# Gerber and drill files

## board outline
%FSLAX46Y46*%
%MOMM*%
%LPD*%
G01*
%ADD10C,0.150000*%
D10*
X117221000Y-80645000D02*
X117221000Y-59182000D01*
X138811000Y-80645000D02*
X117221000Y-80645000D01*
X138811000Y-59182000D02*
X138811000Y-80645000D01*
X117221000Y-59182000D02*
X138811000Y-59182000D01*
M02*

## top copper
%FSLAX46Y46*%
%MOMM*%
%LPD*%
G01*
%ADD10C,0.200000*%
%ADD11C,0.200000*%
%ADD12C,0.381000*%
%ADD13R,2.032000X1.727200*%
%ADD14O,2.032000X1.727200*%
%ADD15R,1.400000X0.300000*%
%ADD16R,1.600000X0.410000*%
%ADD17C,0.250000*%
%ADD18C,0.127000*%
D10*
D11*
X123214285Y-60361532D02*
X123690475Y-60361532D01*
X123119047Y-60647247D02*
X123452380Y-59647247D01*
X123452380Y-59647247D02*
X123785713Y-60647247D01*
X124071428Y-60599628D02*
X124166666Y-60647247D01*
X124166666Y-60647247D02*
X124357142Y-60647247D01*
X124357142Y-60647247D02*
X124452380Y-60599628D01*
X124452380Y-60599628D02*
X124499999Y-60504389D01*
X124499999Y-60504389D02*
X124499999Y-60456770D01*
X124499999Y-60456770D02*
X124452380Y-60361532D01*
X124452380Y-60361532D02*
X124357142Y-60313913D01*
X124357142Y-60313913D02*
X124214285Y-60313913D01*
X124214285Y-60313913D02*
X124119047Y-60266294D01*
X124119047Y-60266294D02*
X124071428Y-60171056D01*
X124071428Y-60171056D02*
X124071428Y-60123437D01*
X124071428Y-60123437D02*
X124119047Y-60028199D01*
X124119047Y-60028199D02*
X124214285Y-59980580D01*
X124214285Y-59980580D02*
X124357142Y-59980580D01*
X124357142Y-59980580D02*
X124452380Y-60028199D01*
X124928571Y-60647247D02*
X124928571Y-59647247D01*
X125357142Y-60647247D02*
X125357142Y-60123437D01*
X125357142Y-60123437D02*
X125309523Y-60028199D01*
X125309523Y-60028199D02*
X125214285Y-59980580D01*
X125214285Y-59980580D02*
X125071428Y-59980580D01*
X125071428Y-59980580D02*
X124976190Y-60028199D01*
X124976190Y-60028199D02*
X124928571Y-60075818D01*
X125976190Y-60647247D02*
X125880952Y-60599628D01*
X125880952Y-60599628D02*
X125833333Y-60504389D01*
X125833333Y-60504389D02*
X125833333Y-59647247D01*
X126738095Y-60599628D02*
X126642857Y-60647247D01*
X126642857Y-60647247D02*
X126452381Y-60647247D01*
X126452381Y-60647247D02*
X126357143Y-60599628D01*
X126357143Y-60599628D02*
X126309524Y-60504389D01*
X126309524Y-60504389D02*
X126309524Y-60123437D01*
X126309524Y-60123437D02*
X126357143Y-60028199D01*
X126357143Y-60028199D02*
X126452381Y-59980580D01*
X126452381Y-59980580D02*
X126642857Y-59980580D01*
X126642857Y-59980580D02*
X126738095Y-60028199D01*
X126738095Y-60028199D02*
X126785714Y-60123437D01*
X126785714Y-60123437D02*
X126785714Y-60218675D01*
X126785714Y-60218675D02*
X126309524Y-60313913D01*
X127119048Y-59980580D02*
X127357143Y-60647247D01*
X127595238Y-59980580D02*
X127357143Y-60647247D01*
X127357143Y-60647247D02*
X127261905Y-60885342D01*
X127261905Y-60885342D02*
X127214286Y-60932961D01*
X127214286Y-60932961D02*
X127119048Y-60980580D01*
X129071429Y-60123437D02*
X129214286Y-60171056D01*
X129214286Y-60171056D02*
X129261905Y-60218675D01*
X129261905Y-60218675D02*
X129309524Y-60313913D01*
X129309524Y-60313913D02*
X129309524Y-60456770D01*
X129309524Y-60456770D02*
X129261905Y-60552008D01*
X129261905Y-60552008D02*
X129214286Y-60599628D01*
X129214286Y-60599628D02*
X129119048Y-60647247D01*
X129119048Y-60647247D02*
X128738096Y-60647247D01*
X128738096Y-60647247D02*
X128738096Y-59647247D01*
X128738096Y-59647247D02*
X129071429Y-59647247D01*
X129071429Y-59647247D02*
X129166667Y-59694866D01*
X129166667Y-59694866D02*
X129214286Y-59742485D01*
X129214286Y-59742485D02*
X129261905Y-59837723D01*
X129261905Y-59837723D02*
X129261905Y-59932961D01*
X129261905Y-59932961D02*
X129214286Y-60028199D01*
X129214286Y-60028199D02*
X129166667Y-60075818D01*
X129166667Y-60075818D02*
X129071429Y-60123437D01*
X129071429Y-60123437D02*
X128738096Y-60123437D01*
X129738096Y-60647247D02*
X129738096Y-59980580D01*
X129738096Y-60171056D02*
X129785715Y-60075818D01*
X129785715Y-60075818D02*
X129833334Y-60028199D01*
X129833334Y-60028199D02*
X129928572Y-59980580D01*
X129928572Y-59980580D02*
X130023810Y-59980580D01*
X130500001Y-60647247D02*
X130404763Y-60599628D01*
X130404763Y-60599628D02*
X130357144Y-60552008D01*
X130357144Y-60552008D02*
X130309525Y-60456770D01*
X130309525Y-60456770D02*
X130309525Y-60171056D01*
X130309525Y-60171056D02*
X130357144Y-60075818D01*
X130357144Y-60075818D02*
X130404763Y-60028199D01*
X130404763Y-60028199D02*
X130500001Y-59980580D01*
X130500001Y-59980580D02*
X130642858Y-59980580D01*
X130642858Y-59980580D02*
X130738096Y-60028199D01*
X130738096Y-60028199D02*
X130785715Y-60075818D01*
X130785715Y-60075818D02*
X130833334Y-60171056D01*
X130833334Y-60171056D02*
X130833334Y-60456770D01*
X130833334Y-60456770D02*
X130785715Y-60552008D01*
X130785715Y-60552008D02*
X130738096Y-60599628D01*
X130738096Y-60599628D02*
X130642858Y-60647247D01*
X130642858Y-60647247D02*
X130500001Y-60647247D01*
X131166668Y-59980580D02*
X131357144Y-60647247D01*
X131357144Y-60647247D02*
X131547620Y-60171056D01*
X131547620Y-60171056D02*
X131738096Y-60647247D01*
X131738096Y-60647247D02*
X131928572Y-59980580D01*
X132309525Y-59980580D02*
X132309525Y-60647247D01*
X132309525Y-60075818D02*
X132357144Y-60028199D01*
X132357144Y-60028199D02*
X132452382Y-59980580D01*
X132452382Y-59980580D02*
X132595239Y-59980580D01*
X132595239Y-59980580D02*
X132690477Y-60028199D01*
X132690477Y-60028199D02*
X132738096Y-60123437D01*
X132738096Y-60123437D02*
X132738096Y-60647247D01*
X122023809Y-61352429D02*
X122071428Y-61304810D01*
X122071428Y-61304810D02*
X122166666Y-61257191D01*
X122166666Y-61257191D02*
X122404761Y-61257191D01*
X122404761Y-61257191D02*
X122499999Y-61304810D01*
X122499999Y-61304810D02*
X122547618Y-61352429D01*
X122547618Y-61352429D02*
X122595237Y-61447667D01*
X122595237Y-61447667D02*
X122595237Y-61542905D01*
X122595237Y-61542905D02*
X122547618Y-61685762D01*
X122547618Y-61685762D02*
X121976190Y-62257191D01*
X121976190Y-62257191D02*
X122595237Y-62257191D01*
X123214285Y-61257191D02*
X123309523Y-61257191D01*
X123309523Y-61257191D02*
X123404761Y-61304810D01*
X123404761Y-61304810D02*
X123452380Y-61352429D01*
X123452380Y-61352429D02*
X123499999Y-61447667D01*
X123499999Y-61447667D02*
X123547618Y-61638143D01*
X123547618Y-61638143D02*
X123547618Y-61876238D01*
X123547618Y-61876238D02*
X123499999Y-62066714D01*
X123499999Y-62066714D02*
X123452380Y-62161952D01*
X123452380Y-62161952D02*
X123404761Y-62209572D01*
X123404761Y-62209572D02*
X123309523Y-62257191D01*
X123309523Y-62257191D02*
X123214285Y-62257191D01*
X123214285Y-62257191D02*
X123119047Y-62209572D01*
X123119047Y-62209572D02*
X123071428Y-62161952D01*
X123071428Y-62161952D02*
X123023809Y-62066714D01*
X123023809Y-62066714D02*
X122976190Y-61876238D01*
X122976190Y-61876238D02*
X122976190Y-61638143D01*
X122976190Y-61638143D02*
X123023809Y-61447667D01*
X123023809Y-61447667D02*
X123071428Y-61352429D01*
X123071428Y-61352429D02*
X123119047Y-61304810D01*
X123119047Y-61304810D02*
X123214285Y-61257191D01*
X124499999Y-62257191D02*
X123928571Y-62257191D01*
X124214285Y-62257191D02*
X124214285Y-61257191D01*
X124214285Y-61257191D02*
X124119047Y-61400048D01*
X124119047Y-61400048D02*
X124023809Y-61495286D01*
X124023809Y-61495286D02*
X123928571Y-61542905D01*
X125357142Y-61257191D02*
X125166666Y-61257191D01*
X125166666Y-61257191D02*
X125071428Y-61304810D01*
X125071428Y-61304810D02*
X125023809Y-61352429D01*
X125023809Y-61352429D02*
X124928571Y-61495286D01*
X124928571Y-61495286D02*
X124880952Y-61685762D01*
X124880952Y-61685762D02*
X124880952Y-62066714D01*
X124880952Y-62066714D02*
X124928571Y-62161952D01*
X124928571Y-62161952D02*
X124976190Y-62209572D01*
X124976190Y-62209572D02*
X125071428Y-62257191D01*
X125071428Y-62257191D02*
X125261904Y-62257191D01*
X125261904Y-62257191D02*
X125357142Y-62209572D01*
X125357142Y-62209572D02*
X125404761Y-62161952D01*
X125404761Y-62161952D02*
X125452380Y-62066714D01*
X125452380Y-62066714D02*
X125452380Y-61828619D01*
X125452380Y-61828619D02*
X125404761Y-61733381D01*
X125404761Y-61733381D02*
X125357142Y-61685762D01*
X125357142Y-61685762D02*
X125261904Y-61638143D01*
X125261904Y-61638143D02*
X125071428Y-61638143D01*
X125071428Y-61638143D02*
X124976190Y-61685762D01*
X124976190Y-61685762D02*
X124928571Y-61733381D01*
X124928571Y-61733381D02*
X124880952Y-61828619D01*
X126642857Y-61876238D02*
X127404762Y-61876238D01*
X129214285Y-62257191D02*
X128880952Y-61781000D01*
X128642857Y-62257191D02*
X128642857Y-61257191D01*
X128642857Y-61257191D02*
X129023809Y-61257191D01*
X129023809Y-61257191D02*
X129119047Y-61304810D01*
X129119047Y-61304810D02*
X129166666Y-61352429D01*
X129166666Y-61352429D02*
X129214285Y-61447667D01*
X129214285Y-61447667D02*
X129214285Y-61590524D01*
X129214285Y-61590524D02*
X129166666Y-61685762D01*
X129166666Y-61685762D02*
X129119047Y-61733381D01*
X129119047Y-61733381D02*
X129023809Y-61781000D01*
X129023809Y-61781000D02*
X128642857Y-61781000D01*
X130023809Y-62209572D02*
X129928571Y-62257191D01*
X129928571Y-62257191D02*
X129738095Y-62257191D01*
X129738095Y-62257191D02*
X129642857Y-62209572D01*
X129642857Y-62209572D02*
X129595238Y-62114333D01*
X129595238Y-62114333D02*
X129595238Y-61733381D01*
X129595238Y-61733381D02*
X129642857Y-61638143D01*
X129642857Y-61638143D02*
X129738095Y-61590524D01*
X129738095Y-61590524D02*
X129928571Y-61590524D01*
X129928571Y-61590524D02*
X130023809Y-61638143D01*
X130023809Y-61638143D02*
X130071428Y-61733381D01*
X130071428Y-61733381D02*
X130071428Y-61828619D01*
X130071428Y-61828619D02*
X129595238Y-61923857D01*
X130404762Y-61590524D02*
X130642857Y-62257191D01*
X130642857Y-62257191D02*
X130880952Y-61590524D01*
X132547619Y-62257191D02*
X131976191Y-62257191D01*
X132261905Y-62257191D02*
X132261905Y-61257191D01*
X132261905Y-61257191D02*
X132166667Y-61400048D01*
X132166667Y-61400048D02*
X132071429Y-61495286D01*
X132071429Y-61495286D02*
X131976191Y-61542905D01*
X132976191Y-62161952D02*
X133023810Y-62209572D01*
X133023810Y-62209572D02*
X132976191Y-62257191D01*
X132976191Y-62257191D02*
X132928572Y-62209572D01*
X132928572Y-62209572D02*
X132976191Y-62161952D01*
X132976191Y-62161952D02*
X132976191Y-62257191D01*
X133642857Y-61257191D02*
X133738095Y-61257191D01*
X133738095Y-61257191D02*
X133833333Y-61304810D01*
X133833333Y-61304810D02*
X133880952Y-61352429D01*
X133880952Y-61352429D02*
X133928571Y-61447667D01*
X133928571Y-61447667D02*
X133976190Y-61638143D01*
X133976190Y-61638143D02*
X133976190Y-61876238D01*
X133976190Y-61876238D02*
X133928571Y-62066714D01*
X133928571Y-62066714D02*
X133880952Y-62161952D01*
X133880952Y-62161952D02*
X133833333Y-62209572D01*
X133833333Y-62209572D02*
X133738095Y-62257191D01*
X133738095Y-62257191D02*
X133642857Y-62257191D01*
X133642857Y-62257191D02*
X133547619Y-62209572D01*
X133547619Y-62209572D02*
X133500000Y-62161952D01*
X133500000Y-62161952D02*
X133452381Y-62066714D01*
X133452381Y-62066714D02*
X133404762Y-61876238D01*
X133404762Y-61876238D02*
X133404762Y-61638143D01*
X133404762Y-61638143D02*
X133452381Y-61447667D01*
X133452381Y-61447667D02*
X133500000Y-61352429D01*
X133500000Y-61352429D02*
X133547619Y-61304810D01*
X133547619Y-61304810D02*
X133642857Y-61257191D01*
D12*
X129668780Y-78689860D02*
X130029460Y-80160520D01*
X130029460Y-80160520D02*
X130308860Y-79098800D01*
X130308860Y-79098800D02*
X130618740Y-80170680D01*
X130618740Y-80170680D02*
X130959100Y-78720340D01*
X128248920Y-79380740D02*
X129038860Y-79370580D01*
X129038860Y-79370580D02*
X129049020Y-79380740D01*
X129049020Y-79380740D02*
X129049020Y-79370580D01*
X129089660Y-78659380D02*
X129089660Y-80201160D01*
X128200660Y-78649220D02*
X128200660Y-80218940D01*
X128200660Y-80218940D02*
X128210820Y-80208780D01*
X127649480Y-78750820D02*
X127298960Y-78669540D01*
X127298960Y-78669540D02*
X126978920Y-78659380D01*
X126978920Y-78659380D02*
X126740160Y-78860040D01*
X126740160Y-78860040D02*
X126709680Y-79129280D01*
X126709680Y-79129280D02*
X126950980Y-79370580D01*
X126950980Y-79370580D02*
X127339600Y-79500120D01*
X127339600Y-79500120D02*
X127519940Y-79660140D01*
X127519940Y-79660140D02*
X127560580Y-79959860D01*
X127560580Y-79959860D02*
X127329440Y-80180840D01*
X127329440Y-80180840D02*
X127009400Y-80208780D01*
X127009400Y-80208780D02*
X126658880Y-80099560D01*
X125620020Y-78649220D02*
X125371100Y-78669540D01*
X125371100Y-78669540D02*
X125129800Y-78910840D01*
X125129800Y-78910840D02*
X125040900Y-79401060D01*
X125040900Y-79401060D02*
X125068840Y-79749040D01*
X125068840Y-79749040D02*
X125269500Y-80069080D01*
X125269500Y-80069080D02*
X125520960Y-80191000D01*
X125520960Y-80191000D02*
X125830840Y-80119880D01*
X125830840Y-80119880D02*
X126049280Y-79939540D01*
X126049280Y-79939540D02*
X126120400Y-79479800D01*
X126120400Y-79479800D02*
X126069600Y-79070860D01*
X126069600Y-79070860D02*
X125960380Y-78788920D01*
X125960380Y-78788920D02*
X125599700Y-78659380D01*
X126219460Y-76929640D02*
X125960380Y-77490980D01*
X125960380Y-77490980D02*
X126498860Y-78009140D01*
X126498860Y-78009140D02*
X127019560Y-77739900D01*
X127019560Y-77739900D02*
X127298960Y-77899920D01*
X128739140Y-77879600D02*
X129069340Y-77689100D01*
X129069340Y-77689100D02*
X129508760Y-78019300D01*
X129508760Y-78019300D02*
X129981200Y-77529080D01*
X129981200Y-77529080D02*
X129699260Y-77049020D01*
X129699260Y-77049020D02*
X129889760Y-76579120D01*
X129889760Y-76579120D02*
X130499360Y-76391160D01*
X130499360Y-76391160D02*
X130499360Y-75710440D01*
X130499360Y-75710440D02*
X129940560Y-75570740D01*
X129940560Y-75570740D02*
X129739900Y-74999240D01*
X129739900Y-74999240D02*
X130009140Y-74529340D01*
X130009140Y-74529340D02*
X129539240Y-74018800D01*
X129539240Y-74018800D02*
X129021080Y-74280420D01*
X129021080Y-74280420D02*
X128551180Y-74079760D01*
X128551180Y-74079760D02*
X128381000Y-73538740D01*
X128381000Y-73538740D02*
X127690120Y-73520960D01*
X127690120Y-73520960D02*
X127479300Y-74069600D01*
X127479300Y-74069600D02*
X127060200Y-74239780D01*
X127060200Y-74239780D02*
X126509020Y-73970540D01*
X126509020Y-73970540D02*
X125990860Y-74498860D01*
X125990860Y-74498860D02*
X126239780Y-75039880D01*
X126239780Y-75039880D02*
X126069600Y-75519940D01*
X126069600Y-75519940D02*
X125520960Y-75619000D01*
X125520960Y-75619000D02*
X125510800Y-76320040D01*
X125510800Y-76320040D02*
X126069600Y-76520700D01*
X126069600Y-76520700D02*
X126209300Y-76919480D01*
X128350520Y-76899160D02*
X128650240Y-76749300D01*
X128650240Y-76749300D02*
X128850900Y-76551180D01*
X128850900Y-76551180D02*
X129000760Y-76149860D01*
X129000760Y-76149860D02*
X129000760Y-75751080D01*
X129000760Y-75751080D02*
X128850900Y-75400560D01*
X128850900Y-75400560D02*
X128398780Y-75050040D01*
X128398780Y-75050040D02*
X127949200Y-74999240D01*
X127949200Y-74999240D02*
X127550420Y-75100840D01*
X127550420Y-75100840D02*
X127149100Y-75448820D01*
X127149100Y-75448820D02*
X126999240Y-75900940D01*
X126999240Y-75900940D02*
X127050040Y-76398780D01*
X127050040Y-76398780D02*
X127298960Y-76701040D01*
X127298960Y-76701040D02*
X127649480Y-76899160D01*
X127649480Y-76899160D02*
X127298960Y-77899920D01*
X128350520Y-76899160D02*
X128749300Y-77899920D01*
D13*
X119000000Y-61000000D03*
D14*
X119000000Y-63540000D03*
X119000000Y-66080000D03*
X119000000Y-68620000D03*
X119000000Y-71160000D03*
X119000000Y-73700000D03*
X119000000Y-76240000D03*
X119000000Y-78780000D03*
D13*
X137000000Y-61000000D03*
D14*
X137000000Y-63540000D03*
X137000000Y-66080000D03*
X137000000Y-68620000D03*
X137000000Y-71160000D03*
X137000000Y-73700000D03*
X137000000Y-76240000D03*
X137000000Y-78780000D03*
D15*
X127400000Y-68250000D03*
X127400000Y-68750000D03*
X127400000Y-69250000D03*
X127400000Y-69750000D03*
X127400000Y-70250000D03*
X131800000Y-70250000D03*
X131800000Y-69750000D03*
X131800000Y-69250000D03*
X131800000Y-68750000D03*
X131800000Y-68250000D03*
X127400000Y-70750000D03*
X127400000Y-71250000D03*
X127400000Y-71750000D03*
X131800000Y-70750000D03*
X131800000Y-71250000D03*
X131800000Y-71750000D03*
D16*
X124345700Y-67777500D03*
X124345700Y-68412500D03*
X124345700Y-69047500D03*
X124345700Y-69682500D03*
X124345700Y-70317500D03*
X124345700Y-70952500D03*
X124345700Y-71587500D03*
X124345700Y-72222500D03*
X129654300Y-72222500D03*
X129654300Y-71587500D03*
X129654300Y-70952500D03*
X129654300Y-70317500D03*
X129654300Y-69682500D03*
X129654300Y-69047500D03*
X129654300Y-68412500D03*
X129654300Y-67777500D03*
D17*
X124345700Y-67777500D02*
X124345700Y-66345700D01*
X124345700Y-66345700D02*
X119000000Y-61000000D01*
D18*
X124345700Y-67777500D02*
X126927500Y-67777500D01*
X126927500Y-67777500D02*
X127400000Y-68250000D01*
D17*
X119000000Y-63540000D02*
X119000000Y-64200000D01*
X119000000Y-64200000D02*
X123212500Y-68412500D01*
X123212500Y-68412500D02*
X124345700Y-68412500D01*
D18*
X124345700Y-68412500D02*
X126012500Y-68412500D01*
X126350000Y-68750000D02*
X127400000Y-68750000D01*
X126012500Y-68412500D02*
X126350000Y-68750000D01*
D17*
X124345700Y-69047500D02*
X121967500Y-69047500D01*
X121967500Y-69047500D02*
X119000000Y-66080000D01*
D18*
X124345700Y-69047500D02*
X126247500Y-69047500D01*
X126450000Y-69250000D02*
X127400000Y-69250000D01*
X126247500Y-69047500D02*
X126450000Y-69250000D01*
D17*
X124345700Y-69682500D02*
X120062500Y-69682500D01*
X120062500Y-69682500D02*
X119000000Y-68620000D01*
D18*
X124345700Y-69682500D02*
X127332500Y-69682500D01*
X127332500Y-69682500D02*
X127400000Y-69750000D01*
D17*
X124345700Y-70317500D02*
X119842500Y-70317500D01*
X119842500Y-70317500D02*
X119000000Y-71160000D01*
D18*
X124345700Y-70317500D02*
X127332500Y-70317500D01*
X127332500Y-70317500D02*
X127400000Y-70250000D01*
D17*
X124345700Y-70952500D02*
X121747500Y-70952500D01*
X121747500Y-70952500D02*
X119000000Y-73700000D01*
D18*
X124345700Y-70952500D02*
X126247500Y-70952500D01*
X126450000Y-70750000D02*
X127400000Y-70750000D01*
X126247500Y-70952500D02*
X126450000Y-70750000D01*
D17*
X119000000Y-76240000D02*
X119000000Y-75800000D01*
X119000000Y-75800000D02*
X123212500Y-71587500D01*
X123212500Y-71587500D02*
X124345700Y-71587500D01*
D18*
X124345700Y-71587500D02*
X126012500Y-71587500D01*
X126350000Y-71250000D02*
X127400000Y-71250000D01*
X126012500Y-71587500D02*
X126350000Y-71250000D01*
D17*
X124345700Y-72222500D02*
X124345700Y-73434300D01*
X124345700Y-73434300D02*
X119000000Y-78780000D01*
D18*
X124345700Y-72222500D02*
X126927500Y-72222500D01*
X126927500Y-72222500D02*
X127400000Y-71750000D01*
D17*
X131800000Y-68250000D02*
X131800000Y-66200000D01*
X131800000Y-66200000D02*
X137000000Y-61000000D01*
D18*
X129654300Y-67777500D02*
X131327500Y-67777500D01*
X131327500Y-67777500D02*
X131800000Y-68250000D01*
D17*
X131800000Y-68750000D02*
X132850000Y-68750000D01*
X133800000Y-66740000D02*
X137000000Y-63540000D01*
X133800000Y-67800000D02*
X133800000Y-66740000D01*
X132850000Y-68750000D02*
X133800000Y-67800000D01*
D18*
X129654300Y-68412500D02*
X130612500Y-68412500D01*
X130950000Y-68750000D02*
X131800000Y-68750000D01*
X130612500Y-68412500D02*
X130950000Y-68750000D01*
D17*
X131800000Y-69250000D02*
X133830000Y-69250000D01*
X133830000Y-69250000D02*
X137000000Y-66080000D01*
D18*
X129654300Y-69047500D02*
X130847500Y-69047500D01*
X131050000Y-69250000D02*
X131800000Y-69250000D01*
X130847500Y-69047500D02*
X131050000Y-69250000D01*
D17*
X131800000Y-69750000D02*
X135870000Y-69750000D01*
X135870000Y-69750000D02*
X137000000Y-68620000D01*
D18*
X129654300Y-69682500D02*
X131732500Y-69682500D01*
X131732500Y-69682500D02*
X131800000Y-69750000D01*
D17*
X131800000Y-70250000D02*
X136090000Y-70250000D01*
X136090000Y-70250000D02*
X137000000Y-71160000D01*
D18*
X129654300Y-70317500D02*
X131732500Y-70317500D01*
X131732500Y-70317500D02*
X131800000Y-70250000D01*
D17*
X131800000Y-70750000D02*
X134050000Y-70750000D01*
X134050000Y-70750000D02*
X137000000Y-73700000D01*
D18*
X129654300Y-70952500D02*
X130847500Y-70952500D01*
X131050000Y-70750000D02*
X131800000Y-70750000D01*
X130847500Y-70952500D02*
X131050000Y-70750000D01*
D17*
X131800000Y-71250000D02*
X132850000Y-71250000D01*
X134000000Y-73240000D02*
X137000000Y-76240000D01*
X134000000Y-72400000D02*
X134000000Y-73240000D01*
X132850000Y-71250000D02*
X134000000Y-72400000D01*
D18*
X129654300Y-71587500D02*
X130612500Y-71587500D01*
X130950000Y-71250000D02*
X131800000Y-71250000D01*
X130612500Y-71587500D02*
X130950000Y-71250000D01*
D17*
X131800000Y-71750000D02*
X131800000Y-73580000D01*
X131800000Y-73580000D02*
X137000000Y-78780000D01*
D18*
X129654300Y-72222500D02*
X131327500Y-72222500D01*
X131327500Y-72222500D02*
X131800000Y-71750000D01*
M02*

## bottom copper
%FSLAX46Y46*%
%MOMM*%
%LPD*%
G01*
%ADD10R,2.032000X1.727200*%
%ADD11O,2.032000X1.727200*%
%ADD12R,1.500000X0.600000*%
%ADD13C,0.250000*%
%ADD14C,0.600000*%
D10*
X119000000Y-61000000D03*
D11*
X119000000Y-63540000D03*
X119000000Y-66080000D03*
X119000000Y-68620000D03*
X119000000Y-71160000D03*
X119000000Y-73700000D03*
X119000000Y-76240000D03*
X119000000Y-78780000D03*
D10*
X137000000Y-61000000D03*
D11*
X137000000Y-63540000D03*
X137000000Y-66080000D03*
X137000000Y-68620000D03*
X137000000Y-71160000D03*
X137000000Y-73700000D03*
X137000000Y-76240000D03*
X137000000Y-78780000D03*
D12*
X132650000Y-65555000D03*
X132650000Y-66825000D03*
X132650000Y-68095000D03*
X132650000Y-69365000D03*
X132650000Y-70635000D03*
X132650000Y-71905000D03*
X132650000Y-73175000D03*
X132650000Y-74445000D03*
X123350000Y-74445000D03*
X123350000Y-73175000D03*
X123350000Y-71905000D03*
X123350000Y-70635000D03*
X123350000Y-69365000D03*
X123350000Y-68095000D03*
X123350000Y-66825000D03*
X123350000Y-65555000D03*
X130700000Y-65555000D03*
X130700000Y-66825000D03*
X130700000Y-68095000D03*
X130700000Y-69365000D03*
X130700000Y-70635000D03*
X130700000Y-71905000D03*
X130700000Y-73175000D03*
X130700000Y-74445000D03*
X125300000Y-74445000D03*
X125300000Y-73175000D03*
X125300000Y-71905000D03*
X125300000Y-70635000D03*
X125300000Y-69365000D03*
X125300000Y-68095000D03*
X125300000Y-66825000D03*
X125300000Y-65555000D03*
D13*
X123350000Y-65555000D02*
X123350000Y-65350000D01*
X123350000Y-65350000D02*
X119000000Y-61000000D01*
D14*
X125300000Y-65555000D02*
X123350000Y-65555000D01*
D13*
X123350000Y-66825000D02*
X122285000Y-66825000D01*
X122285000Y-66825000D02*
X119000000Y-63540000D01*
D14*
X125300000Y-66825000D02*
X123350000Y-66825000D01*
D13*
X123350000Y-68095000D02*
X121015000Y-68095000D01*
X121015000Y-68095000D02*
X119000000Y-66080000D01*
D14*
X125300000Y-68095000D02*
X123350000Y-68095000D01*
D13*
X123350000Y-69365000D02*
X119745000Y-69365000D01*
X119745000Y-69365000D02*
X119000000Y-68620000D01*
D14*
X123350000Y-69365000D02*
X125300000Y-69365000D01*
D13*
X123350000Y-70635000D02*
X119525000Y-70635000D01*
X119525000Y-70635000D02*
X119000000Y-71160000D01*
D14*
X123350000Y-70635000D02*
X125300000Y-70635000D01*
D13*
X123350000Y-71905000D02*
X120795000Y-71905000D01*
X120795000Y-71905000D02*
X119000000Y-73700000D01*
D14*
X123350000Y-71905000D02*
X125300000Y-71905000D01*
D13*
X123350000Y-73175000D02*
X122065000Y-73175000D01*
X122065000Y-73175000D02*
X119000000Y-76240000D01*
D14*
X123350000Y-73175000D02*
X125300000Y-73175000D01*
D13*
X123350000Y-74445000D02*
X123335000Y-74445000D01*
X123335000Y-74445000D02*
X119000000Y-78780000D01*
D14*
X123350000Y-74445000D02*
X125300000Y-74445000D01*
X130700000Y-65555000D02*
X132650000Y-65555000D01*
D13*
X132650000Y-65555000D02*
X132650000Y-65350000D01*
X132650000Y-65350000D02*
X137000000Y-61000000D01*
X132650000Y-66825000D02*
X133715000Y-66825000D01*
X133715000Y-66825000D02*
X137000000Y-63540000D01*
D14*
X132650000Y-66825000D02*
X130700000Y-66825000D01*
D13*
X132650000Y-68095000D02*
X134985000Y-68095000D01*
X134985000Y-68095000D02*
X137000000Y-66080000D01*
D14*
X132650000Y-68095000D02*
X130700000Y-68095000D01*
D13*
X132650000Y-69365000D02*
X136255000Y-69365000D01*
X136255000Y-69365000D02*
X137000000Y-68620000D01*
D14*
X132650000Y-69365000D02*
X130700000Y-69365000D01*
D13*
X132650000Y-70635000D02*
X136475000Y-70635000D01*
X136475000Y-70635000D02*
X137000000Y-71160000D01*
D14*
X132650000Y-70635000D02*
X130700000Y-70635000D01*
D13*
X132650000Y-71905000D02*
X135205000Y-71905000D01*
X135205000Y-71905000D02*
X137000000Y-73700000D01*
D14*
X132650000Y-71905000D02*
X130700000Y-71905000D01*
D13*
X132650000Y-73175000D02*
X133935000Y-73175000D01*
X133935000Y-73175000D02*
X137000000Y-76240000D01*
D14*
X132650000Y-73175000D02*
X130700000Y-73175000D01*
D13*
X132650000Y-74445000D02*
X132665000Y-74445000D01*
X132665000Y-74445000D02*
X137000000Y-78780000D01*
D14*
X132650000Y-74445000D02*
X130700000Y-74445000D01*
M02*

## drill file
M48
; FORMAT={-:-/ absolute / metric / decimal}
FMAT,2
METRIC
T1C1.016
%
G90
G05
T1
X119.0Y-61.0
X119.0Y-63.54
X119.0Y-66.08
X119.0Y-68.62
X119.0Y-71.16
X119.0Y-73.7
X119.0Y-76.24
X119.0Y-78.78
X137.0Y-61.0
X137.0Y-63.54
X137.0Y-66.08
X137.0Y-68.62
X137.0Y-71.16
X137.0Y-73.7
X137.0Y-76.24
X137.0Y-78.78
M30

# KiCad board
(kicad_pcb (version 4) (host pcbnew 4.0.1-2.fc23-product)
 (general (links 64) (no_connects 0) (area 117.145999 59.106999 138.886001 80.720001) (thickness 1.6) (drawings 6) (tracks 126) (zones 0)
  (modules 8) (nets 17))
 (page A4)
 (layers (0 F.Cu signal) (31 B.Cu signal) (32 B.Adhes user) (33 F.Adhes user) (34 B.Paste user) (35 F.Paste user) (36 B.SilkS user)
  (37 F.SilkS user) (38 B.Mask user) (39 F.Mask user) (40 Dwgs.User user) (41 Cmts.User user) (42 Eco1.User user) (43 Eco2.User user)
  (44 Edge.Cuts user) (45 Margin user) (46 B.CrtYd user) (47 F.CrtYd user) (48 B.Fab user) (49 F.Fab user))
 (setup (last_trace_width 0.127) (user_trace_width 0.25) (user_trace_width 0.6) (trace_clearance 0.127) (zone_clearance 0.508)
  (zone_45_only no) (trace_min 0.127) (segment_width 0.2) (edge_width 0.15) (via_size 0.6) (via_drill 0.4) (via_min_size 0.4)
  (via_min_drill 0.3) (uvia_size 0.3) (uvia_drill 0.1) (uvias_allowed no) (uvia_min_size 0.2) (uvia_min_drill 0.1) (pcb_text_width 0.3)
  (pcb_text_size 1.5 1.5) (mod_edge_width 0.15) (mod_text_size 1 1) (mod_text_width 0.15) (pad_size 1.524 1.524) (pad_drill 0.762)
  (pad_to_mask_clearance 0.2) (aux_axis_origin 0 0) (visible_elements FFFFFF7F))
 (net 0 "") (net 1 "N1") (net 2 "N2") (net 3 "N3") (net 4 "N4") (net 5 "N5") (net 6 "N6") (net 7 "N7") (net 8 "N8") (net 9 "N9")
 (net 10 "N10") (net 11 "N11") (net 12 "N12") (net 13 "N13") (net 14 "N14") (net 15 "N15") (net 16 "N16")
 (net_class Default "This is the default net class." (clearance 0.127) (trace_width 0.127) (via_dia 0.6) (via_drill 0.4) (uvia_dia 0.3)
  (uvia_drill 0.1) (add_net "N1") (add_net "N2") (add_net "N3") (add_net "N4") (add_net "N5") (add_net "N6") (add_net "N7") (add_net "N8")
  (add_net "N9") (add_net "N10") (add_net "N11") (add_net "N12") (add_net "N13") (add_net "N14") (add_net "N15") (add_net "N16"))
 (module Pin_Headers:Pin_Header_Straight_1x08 (layer F.Cu) (at 119 61)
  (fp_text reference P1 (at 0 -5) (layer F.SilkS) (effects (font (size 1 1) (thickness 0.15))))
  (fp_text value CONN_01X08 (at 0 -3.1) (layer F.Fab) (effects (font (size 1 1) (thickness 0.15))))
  (pad 1 thru_hole rect (at 0 0) (size 2.032 1.7272) (drill 1.016) (layers *.Cu *.Mask F.SilkS) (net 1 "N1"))
  (pad 2 thru_hole oval (at 0 2.54) (size 2.032 1.7272) (drill 1.016) (layers *.Cu *.Mask F.SilkS) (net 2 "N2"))
  (pad 3 thru_hole oval (at 0 5.08) (size 2.032 1.7272) (drill 1.016) (layers *.Cu *.Mask F.SilkS) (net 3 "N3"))
  (pad 4 thru_hole oval (at 0 7.62) (size 2.032 1.7272) (drill 1.016) (layers *.Cu *.Mask F.SilkS) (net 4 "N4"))
  (pad 5 thru_hole oval (at 0 10.16) (size 2.032 1.7272) (drill 1.016) (layers *.Cu *.Mask F.SilkS) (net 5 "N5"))
  (pad 6 thru_hole oval (at 0 12.7) (size 2.032 1.7272) (drill 1.016) (layers *.Cu *.Mask F.SilkS) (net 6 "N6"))
  (pad 7 thru_hole oval (at 0 15.24) (size 2.032 1.7272) (drill 1.016) (layers *.Cu *.Mask F.SilkS) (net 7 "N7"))
  (pad 8 thru_hole oval (at 0 17.78) (size 2.032 1.7272) (drill 1.016) (layers *.Cu *.Mask F.SilkS) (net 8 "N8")))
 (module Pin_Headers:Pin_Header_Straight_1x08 (layer F.Cu) (at 137 61)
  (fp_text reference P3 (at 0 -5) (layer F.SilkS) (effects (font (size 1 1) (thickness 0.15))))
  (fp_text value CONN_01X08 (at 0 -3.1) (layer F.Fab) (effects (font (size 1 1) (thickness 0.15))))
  (pad 1 thru_hole rect (at 0 0) (size 2.032 1.7272) (drill 1.016) (layers *.Cu *.Mask F.SilkS) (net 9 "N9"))
  (pad 2 thru_hole oval (at 0 2.54) (size 2.032 1.7272) (drill 1.016) (layers *.Cu *.Mask F.SilkS) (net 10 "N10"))
  (pad 3 thru_hole oval (at 0 5.08) (size 2.032 1.7272) (drill 1.016) (layers *.Cu *.Mask F.SilkS) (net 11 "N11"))
  (pad 4 thru_hole oval (at 0 7.62) (size 2.032 1.7272) (drill 1.016) (layers *.Cu *.Mask F.SilkS) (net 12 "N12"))
  (pad 5 thru_hole oval (at 0 10.16) (size 2.032 1.7272) (drill 1.016) (layers *.Cu *.Mask F.SilkS) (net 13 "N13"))
  (pad 6 thru_hole oval (at 0 12.7) (size 2.032 1.7272) (drill 1.016) (layers *.Cu *.Mask F.SilkS) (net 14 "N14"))
  (pad 7 thru_hole oval (at 0 15.24) (size 2.032 1.7272) (drill 1.016) (layers *.Cu *.Mask F.SilkS) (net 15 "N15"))
  (pad 8 thru_hole oval (at 0 17.78) (size 2.032 1.7272) (drill 1.016) (layers *.Cu *.Mask F.SilkS) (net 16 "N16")))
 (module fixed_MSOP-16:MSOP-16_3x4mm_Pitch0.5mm (layer F.Cu) (at 129.6 70)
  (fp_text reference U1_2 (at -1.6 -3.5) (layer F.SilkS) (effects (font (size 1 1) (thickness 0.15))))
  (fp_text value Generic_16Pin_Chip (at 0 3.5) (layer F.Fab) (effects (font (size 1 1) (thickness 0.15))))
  (pad 1 smd rect (at -2.2 -1.75) (size 1.4 0.3) (layers F.Cu F.Paste F.Mask) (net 1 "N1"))
  (pad 2 smd rect (at -2.2 -1.25) (size 1.4 0.3) (layers F.Cu F.Paste F.Mask) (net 2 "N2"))
  (pad 3 smd rect (at -2.2 -0.75) (size 1.4 0.3) (layers F.Cu F.Paste F.Mask) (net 3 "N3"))
  (pad 4 smd rect (at -2.2 -0.25) (size 1.4 0.3) (layers F.Cu F.Paste F.Mask) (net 4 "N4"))
  (pad 5 smd rect (at -2.2 0.25) (size 1.4 0.3) (layers F.Cu F.Paste F.Mask) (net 5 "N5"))
  (pad 12 smd rect (at 2.2 0.25) (size 1.4 0.3) (layers F.Cu F.Paste F.Mask) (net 13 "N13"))
  (pad 13 smd rect (at 2.2 -0.25) (size 1.4 0.3) (layers F.Cu F.Paste F.Mask) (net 12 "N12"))
  (pad 14 smd rect (at 2.2 -0.75) (size 1.4 0.3) (layers F.Cu F.Paste F.Mask) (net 11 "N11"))
  (pad 15 smd rect (at 2.2 -1.25) (size 1.4 0.3) (layers F.Cu F.Paste F.Mask) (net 10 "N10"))
  (pad 16 smd rect (at 2.2 -1.75) (size 1.4 0.3) (layers F.Cu F.Paste F.Mask) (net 9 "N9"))
  (pad 6 smd rect (at -2.2 0.75) (size 1.4 0.3) (layers F.Cu F.Paste F.Mask) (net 6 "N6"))
  (pad 7 smd rect (at -2.2 1.25) (size 1.4 0.3) (layers F.Cu F.Paste F.Mask) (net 7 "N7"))
  (pad 8 smd rect (at -2.2 1.75) (size 1.4 0.3) (layers F.Cu F.Paste F.Mask) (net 8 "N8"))
  (pad 11 smd rect (at 2.2 0.75) (size 1.4 0.3) (layers F.Cu F.Paste F.Mask) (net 14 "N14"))
  (pad 10 smd rect (at 2.2 1.25) (size 1.4 0.3) (layers F.Cu F.Paste F.Mask) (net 15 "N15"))
  (pad 9 smd rect (at 2.2 1.75) (size 1.4 0.3) (layers F.Cu F.Paste F.Mask) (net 16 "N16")))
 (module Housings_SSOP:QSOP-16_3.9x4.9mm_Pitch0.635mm (layer F.Cu) (at 127 70)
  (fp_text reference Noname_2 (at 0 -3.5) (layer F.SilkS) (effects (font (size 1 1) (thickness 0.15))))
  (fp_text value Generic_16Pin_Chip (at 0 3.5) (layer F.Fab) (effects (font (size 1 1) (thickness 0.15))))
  (pad 1 smd rect (at -2.6543 -2.2225) (size 1.6 0.41) (layers F.Cu F.Paste F.Mask) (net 1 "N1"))
  (pad 2 smd rect (at -2.6543 -1.5875) (size 1.6 0.41) (layers F.Cu F.Paste F.Mask) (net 2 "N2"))
  (pad 3 smd rect (at -2.6543 -0.9525) (size 1.6 0.41) (layers F.Cu F.Paste F.Mask) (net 3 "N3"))
  (pad 4 smd rect (at -2.6543 -0.3175) (size 1.6 0.41) (layers F.Cu F.Paste F.Mask) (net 4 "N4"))
  (pad 5 smd rect (at -2.6543 0.3175) (size 1.6 0.41) (layers F.Cu F.Paste F.Mask) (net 5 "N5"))
  (pad 6 smd rect (at -2.6543 0.9525) (size 1.6 0.41) (layers F.Cu F.Paste F.Mask) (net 6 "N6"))
  (pad 7 smd rect (at -2.6543 1.5875) (size 1.6 0.41) (layers F.Cu F.Paste F.Mask) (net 7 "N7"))
  (pad 8 smd rect (at -2.6543 2.2225) (size 1.6 0.41) (layers F.Cu F.Paste F.Mask) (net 8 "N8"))
  (pad 9 smd rect (at 2.6543 2.2225) (size 1.6 0.41) (layers F.Cu F.Paste F.Mask) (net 16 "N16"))
  (pad 10 smd rect (at 2.6543 1.5875) (size 1.6 0.41) (layers F.Cu F.Paste F.Mask) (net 15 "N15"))
  (pad 11 smd rect (at 2.6543 0.9525) (size 1.6 0.41) (layers F.Cu F.Paste F.Mask) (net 14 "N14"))
  (pad 12 smd rect (at 2.6543 0.3175) (size 1.6 0.41) (layers F.Cu F.Paste F.Mask) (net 13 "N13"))
  (pad 13 smd rect (at 2.6543 -0.3175) (size 1.6 0.41) (layers F.Cu F.Paste F.Mask) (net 12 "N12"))
  (pad 14 smd rect (at 2.6543 -0.9525) (size 1.6 0.41) (layers F.Cu F.Paste F.Mask) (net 11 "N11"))
  (pad 15 smd rect (at 2.6543 -1.5875) (size 1.6 0.41) (layers F.Cu F.Paste F.Mask) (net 10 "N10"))
  (pad 16 smd rect (at 2.6543 -2.2225) (size 1.6 0.41) (layers F.Cu F.Paste F.Mask) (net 9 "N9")))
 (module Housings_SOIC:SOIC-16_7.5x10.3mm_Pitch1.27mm (layer B.Cu) (at 128 70 180)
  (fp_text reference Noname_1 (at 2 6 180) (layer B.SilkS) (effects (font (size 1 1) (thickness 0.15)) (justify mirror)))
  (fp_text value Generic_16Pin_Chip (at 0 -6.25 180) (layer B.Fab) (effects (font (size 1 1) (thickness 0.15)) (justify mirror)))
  (pad 1 smd rect (at -4.65 4.445 180) (size 1.5 0.6) (layers B.Cu B.Paste B.Mask) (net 9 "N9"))
  (pad 2 smd rect (at -4.65 3.175 180) (size 1.5 0.6) (layers B.Cu B.Paste B.Mask) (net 10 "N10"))
  (pad 3 smd rect (at -4.65 1.905 180) (size 1.5 0.6) (layers B.Cu B.Paste B.Mask) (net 11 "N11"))
  (pad 4 smd rect (at -4.65 0.635 180) (size 1.5 0.6) (layers B.Cu B.Paste B.Mask) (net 12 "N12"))
  (pad 5 smd rect (at -4.65 -0.635 180) (size 1.5 0.6) (layers B.Cu B.Paste B.Mask) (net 13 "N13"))
  (pad 6 smd rect (at -4.65 -1.905 180) (size 1.5 0.6) (layers B.Cu B.Paste B.Mask) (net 14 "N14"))
  (pad 7 smd rect (at -4.65 -3.175 180) (size 1.5 0.6) (layers B.Cu B.Paste B.Mask) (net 15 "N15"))
  (pad 8 smd rect (at -4.65 -4.445 180) (size 1.5 0.6) (layers B.Cu B.Paste B.Mask) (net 16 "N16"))
  (pad 9 smd rect (at 4.65 -4.445 180) (size 1.5 0.6) (layers B.Cu B.Paste B.Mask) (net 8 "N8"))
  (pad 10 smd rect (at 4.65 -3.175 180) (size 1.5 0.6) (layers B.Cu B.Paste B.Mask) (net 7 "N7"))
  (pad 11 smd rect (at 4.65 -1.905 180) (size 1.5 0.6) (layers B.Cu B.Paste B.Mask) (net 6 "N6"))
  (pad 12 smd rect (at 4.65 -0.635 180) (size 1.5 0.6) (layers B.Cu B.Paste B.Mask) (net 5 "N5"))
  (pad 13 smd rect (at 4.65 0.635 180) (size 1.5 0.6) (layers B.Cu B.Paste B.Mask) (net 4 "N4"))
  (pad 14 smd rect (at 4.65 1.905 180) (size 1.5 0.6) (layers B.Cu B.Paste B.Mask) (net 3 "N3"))
  (pad 15 smd rect (at 4.65 3.175 180) (size 1.5 0.6) (layers B.Cu B.Paste B.Mask) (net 2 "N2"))
  (pad 16 smd rect (at 4.65 4.445 180) (size 1.5 0.6) (layers B.Cu B.Paste B.Mask) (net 1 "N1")))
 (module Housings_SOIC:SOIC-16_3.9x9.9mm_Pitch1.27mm (layer B.Cu) (at 128 70 180)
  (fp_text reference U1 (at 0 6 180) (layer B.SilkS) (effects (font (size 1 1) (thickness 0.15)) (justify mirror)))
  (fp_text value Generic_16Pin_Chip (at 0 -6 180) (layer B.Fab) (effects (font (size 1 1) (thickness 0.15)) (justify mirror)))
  (pad 1 smd rect (at -2.7 4.445 180) (size 1.5 0.6) (layers B.Cu B.Paste B.Mask) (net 9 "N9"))
  (pad 2 smd rect (at -2.7 3.175 180) (size 1.5 0.6) (layers B.Cu B.Paste B.Mask) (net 10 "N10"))
  (pad 3 smd rect (at -2.7 1.905 180) (size 1.5 0.6) (layers B.Cu B.Paste B.Mask) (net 11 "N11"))
  (pad 4 smd rect (at -2.7 0.635 180) (size 1.5 0.6) (layers B.Cu B.Paste B.Mask) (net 12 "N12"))
  (pad 5 smd rect (at -2.7 -0.635 180) (size 1.5 0.6) (layers B.Cu B.Paste B.Mask) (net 13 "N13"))
  (pad 6 smd rect (at -2.7 -1.905 180) (size 1.5 0.6) (layers B.Cu B.Paste B.Mask) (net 14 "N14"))
  (pad 7 smd rect (at -2.7 -3.175 180) (size 1.5 0.6) (layers B.Cu B.Paste B.Mask) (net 15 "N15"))
  (pad 8 smd rect (at -2.7 -4.445 180) (size 1.5 0.6) (layers B.Cu B.Paste B.Mask) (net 16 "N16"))
  (pad 9 smd rect (at 2.7 -4.445 180) (size 1.5 0.6) (layers B.Cu B.Paste B.Mask) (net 8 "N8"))
  (pad 10 smd rect (at 2.7 -3.175 180) (size 1.5 0.6) (layers B.Cu B.Paste B.Mask) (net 7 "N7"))
  (pad 11 smd rect (at 2.7 -1.905 180) (size 1.5 0.6) (layers B.Cu B.Paste B.Mask) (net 6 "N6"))
  (pad 12 smd rect (at 2.7 -0.635 180) (size 1.5 0.6) (layers B.Cu B.Paste B.Mask) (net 5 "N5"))
  (pad 13 smd rect (at 2.7 0.635 180) (size 1.5 0.6) (layers B.Cu B.Paste B.Mask) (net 4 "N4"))
  (pad 14 smd rect (at 2.7 1.905 180) (size 1.5 0.6) (layers B.Cu B.Paste B.Mask) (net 3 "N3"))
  (pad 15 smd rect (at 2.7 3.175 180) (size 1.5 0.6) (layers B.Cu B.Paste B.Mask) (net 2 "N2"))
  (pad 16 smd rect (at 2.7 4.445 180) (size 1.5 0.6) (layers B.Cu B.Paste B.Mask) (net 1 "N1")))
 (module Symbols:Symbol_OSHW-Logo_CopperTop (layer F.Cu) (at 128 76)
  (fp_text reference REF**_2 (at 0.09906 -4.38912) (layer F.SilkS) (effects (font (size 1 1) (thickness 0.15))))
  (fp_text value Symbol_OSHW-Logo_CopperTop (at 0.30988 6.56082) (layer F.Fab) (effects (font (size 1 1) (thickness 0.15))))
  (fp_line (start 1.66878 2.68986) (end 2.02946 4.16052) (layer F.Cu) (width 0.381))
  (fp_line (start 2.02946 4.16052) (end 2.30886 3.0988) (layer F.Cu) (width 0.381))
  (fp_line (start 2.30886 3.0988) (end 2.61874 4.17068) (layer F.Cu) (width 0.381))
  (fp_line (start 2.61874 4.17068) (end 2.9591 2.72034) (layer F.Cu) (width 0.381))
  (fp_line (start 0.24892 3.38074) (end 1.03886 3.37058) (layer F.Cu) (width 0.381))
  (fp_line (start 1.03886 3.37058) (end 1.04902 3.38074) (layer F.Cu) (width 0.381))
  (fp_line (start 1.04902 3.38074) (end 1.04902 3.37058) (layer F.Cu) (width 0.381))
  (fp_line (start 1.08966 2.65938) (end 1.08966 4.20116) (layer F.Cu) (width 0.381))
  (fp_line (start 0.20066 2.64922) (end 0.20066 4.21894) (layer F.Cu) (width 0.381))
  (fp_line (start 0.20066 4.21894) (end 0.21082 4.20878) (layer F.Cu) (width 0.381))
  (fp_line (start -0.35052 2.75082) (end -0.70104 2.66954) (layer F.Cu) (width 0.381))
  (fp_line (start -0.70104 2.66954) (end -1.02108 2.65938) (layer F.Cu) (width 0.381))
  (fp_line (start -1.02108 2.65938) (end -1.25984 2.86004) (layer F.Cu) (width 0.381))
  (fp_line (start -1.25984 2.86004) (end -1.29032 3.12928) (layer F.Cu) (width 0.381))
  (fp_line (start -1.29032 3.12928) (end -1.04902 3.37058) (layer F.Cu) (width 0.381))
  (fp_line (start -1.04902 3.37058) (end -0.6604 3.50012) (layer F.Cu) (width 0.381))
  (fp_line (start -0.6604 3.50012) (end -0.48006 3.66014) (layer F.Cu) (width 0.381))
  (fp_line (start -0.48006 3.66014) (end -0.43942 3.95986) (layer F.Cu) (width 0.381))
  (fp_line (start -0.43942 3.95986) (end -0.67056 4.18084) (layer F.Cu) (width 0.381))
  (fp_line (start -0.67056 4.18084) (end -0.9906 4.20878) (layer F.Cu) (width 0.381))
  (fp_line (start -0.9906 4.20878) (end -1.34112 4.09956) (layer F.Cu) (width 0.381))
  (fp_line (start -2.37998 2.64922) (end -2.6289 2.66954) (layer F.Cu) (width 0.381))
  (fp_line (start -2.6289 2.66954) (end -2.8702 2.91084) (layer F.Cu) (width 0.381))
  (fp_line (start -2.8702 2.91084) (end -2.9591 3.40106) (layer F.Cu) (width 0.381))
  (fp_line (start -2.9591 3.40106) (end -2.93116 3.74904) (layer F.Cu) (width 0.381))
  (fp_line (start -2.93116 3.74904) (end -2.7305 4.06908) (layer F.Cu) (width 0.381))
  (fp_line (start -2.7305 4.06908) (end -2.47904 4.191) (layer F.Cu) (width 0.381))
  (fp_line (start -2.47904 4.191) (end -2.16916 4.11988) (layer F.Cu) (width 0.381))
  (fp_line (start -2.16916 4.11988) (end -1.95072 3.93954) (layer F.Cu) (width 0.381))
  (fp_line (start -1.95072 3.93954) (end -1.8796 3.4798) (layer F.Cu) (width 0.381))
  (fp_line (start -1.8796 3.4798) (end -1.9304 3.07086) (layer F.Cu) (width 0.381))
  (fp_line (start -1.9304 3.07086) (end -2.03962 2.78892) (layer F.Cu) (width 0.381))
  (fp_line (start -2.03962 2.78892) (end -2.4003 2.65938) (layer F.Cu) (width 0.381))
  (fp_line (start -1.78054 0.92964) (end -2.03962 1.49098) (layer F.Cu) (width 0.381))
  (fp_line (start -2.03962 1.49098) (end -1.50114 2.00914) (layer F.Cu) (width 0.381))
  (fp_line (start -1.50114 2.00914) (end -0.98044 1.7399) (layer F.Cu) (width 0.381))
  (fp_line (start -0.98044 1.7399) (end -0.70104 1.89992) (layer F.Cu) (width 0.381))
  (fp_line (start 0.73914 1.8796) (end 1.06934 1.6891) (layer F.Cu) (width 0.381))
  (fp_line (start 1.06934 1.6891) (end 1.50876 2.0193) (layer F.Cu) (width 0.381))
  (fp_line (start 1.50876 2.0193) (end 1.9812 1.52908) (layer F.Cu) (width 0.381))
  (fp_line (start 1.9812 1.52908) (end 1.69926 1.04902) (layer F.Cu) (width 0.381))
  (fp_line (start 1.69926 1.04902) (end 1.88976 0.57912) (layer F.Cu) (width 0.381))
  (fp_line (start 1.88976 0.57912) (end 2.49936 0.39116) (layer F.Cu) (width 0.381))
  (fp_line (start 2.49936 0.39116) (end 2.49936 -0.28956) (layer F.Cu) (width 0.381))
  (fp_line (start 2.49936 -0.28956) (end 1.94056 -0.42926) (layer F.Cu) (width 0.381))
  (fp_line (start 1.94056 -0.42926) (end 1.7399 -1.00076) (layer F.Cu) (width 0.381))
  (fp_line (start 1.7399 -1.00076) (end 2.00914 -1.47066) (layer F.Cu) (width 0.381))
  (fp_line (start 2.00914 -1.47066) (end 1.53924 -1.9812) (layer F.Cu) (width 0.381))
  (fp_line (start 1.53924 -1.9812) (end 1.02108 -1.71958) (layer F.Cu) (width 0.381))
  (fp_line (start 1.02108 -1.71958) (end 0.55118 -1.92024) (layer F.Cu) (width 0.381))
  (fp_line (start 0.55118 -1.92024) (end 0.381 -2.46126) (layer F.Cu) (width 0.381))
  (fp_line (start 0.381 -2.46126) (end -0.30988 -2.47904) (layer F.Cu) (width 0.381))
  (fp_line (start -0.30988 -2.47904) (end -0.5207 -1.9304) (layer F.Cu) (width 0.381))
  (fp_line (start -0.5207 -1.9304) (end -0.9398 -1.76022) (layer F.Cu) (width 0.381))
  (fp_line (start -0.9398 -1.76022) (end -1.49098 -2.02946) (layer F.Cu) (width 0.381))
  (fp_line (start -1.49098 -2.02946) (end -2.00914 -1.50114) (layer F.Cu) (width 0.381))
  (fp_line (start -2.00914 -1.50114) (end -1.76022 -0.96012) (layer F.Cu) (width 0.381))
  (fp_line (start -1.76022 -0.96012) (end -1.9304 -0.48006) (layer F.Cu) (width 0.381))
  (fp_line (start -1.9304 -0.48006) (end -2.47904 -0.381) (layer F.Cu) (width 0.381))
  (fp_line (start -2.47904 -0.381) (end -2.4892 0.32004) (layer F.Cu) (width 0.381))
  (fp_line (start -2.4892 0.32004) (end -1.9304 0.5207) (layer F.Cu) (width 0.381))
  (fp_line (start -1.9304 0.5207) (end -1.7907 0.91948) (layer F.Cu) (width 0.381))
  (fp_line (start 0.35052 0.89916) (end 0.65024 0.7493) (layer F.Cu) (width 0.381))
  (fp_line (start 0.65024 0.7493) (end 0.8509 0.55118) (layer F.Cu) (width 0.381))
  (fp_line (start 0.8509 0.55118) (end 1.00076 0.14986) (layer F.Cu) (width 0.381))
  (fp_line (start 1.00076 0.14986) (end 1.00076 -0.24892) (layer F.Cu) (width 0.381))
  (fp_line (start 1.00076 -0.24892) (end 0.8509 -0.59944) (layer F.Cu) (width 0.381))
  (fp_line (start 0.8509 -0.59944) (end 0.39878 -0.94996) (layer F.Cu) (width 0.381))
  (fp_line (start 0.39878 -0.94996) (end -0.0508 -1.00076) (layer F.Cu) (width 0.381))
  (fp_line (start -0.0508 -1.00076) (end -0.44958 -0.89916) (layer F.Cu) (width 0.381))
  (fp_line (start -0.44958 -0.89916) (end -0.8509 -0.55118) (layer F.Cu) (width 0.381))
  (fp_line (start -0.8509 -0.55118) (end -1.00076 -0.09906) (layer F.Cu) (width 0.381))
  (fp_line (start -1.00076 -0.09906) (end -0.94996 0.39878) (layer F.Cu) (width 0.381))
  (fp_line (start -0.94996 0.39878) (end -0.70104 0.70104) (layer F.Cu) (width 0.381))
  (fp_line (start -0.70104 0.70104) (end -0.35052 0.89916) (layer F.Cu) (width 0.381))
  (fp_line (start -0.35052 0.89916) (end -0.70104 1.89992) (layer F.Cu) (width 0.381))
  (fp_line (start 0.35052 0.89916) (end 0.7493 1.89992) (layer F.Cu) (width 0.381)))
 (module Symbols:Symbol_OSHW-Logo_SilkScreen (layer F.Cu) (at 128 76)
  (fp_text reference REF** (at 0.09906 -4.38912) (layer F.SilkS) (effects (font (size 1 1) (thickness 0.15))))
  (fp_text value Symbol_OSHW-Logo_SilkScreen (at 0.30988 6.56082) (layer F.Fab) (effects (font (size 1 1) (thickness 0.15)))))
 (gr_line (start 117.221 80.645) (end 117.221 59.182) (angle 90) (layer Edge.Cuts) (width 0.15))
 (gr_line (start 138.811 80.645) (end 117.221 80.645) (angle 90) (layer Edge.Cuts) (width 0.15))
 (gr_line (start 138.811 59.182) (end 138.811 80.645) (angle 90) (layer Edge.Cuts) (width 0.15))
 (gr_line (start 117.221 59.182) (end 138.811 59.182) (angle 90) (layer Edge.Cuts) (width 0.15))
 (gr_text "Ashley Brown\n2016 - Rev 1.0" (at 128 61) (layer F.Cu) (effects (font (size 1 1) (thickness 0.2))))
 (segment (start 124.3457 67.7775) (end 124.3457 66.3457) (width 0.25) (layer F.Cu) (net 1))
 (segment (start 124.3457 66.3457) (end 119 61) (width 0.25) (layer F.Cu) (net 1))
 (segment (start 123.35 65.555) (end 123.35 65.35) (width 0.25) (layer B.Cu) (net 1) (status 30))
 (segment (start 123.35 65.35) (end 119 61) (width 0.25) (layer B.Cu) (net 1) (status 10))
 (segment (start 125.3 65.555) (end 123.35 65.555) (width 0.6) (layer B.Cu) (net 1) (status 20))
 (segment (start 124.3457 67.7775) (end 126.9275 67.7775) (width 0.127) (layer F.Cu) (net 1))
 (segment (start 126.9275 67.7775) (end 127.4 68.25) (width 0.127) (layer F.Cu) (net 1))
 (segment (start 119 63.54) (end 119 64.2) (width 0.25) (layer F.Cu) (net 2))
 (segment (start 119 64.2) (end 123.2125 68.4125) (width 0.25) (layer F.Cu) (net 2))
 (segment (start 123.2125 68.4125) (end 124.3457 68.4125) (width 0.25) (layer F.Cu) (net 2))
 (segment (start 123.35 66.825) (end 122.285 66.825) (width 0.25) (layer B.Cu) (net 2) (status 10))
 (segment (start 122.285 66.825) (end 119 63.54) (width 0.25) (layer B.Cu) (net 2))
 (segment (start 125.3 66.825) (end 123.35 66.825) (width 0.6) (layer B.Cu) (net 2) (status 20))
 (segment (start 124.3457 68.4125) (end 126.0125 68.4125) (width 0.127) (layer F.Cu) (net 2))
 (segment (start 126.35 68.75) (end 127.4 68.75) (width 0.127) (layer F.Cu) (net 2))
 (segment (start 126.0125 68.4125) (end 126.35 68.75) (width 0.127) (layer F.Cu) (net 2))
 (segment (start 124.3457 69.0475) (end 121.9675 69.0475) (width 0.25) (layer F.Cu) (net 3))
 (segment (start 121.9675 69.0475) (end 119 66.08) (width 0.25) (layer F.Cu) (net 3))
 (segment (start 123.35 68.095) (end 121.015 68.095) (width 0.25) (layer B.Cu) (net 3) (status 10))
 (segment (start 121.015 68.095) (end 119 66.08) (width 0.25) (layer B.Cu) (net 3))
 (segment (start 125.3 68.095) (end 123.35 68.095) (width 0.6) (layer B.Cu) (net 3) (status 20))
 (segment (start 124.3457 69.0475) (end 126.2475 69.0475) (width 0.127) (layer F.Cu) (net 3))
 (segment (start 126.45 69.25) (end 127.4 69.25) (width 0.127) (layer F.Cu) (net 3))
 (segment (start 126.2475 69.0475) (end 126.45 69.25) (width 0.127) (layer F.Cu) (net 3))
 (segment (start 124.3457 69.6825) (end 120.0625 69.6825) (width 0.25) (layer F.Cu) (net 4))
 (segment (start 120.0625 69.6825) (end 119 68.62) (width 0.25) (layer F.Cu) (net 4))
 (segment (start 123.35 69.365) (end 119.745 69.365) (width 0.25) (layer B.Cu) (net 4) (status 10))
 (segment (start 119.745 69.365) (end 119 68.62) (width 0.25) (layer B.Cu) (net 4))
 (segment (start 123.35 69.365) (end 125.3 69.365) (width 0.6) (layer B.Cu) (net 4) (status 10))
 (segment (start 124.3457 69.6825) (end 127.3325 69.6825) (width 0.127) (layer F.Cu) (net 4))
 (segment (start 127.3325 69.6825) (end 127.4 69.75) (width 0.127) (layer F.Cu) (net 4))
 (segment (start 124.3457 70.3175) (end 119.8425 70.3175) (width 0.25) (layer F.Cu) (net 5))
 (segment (start 119.8425 70.3175) (end 119 71.16) (width 0.25) (layer F.Cu) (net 5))
 (segment (start 123.35 70.635) (end 119.525 70.635) (width 0.25) (layer B.Cu) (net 5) (status 10))
 (segment (start 119.525 70.635) (end 119 71.16) (width 0.25) (layer B.Cu) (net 5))
 (segment (start 123.35 70.635) (end 125.3 70.635) (width 0.6) (layer B.Cu) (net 5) (status 10))
 (segment (start 124.3457 70.3175) (end 127.3325 70.3175) (width 0.127) (layer F.Cu) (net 5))
 (segment (start 127.3325 70.3175) (end 127.4 70.25) (width 0.127) (layer F.Cu) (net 5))
 (segment (start 124.3457 70.9525) (end 121.7475 70.9525) (width 0.25) (layer F.Cu) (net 6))
 (segment (start 121.7475 70.9525) (end 119 73.7) (width 0.25) (layer F.Cu) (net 6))
 (segment (start 123.35 71.905) (end 120.795 71.905) (width 0.25) (layer B.Cu) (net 6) (status 10))
 (segment (start 120.795 71.905) (end 119 73.7) (width 0.25) (layer B.Cu) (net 6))
 (segment (start 123.35 71.905) (end 125.3 71.905) (width 0.6) (layer B.Cu) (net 6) (status 10))
 (segment (start 124.3457 70.9525) (end 126.2475 70.9525) (width 0.127) (layer F.Cu) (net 6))
 (segment (start 126.45 70.75) (end 127.4 70.75) (width 0.127) (layer F.Cu) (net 6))
 (segment (start 126.2475 70.9525) (end 126.45 70.75) (width 0.127) (layer F.Cu) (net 6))
 (segment (start 119 76.24) (end 119 75.8) (width 0.25) (layer F.Cu) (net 7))
 (segment (start 119 75.8) (end 123.2125 71.5875) (width 0.25) (layer F.Cu) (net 7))
 (segment (start 123.2125 71.5875) (end 124.3457 71.5875) (width 0.25) (layer F.Cu) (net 7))
 (segment (start 123.35 73.175) (end 122.065 73.175) (width 0.25) (layer B.Cu) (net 7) (status 10))
 (segment (start 122.065 73.175) (end 119 76.24) (width 0.25) (layer B.Cu) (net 7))
 (segment (start 123.35 73.175) (end 125.3 73.175) (width 0.6) (layer B.Cu) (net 7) (status 10))
 (segment (start 124.3457 71.5875) (end 126.0125 71.5875) (width 0.127) (layer F.Cu) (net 7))
 (segment (start 126.35 71.25) (end 127.4 71.25) (width 0.127) (layer F.Cu) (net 7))
 (segment (start 126.0125 71.5875) (end 126.35 71.25) (width 0.127) (layer F.Cu) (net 7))
 (segment (start 124.3457 72.2225) (end 124.3457 73.4343) (width 0.25) (layer F.Cu) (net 8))
 (segment (start 124.3457 73.4343) (end 119 78.78) (width 0.25) (layer F.Cu) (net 8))
 (segment (start 123.35 74.445) (end 123.335 74.445) (width 0.25) (layer B.Cu) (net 8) (status 30))
 (segment (start 123.335 74.445) (end 119 78.78) (width 0.25) (layer B.Cu) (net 8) (status 10))
 (segment (start 123.35 74.445) (end 125.3 74.445) (width 0.6) (layer B.Cu) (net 8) (status 10))
 (segment (start 124.3457 72.2225) (end 126.9275 72.2225) (width 0.127) (layer F.Cu) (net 8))
 (segment (start 126.9275 72.2225) (end 127.4 71.75) (width 0.127) (layer F.Cu) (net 8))
 (segment (start 130.7 65.555) (end 132.65 65.555) (width 0.6) (layer B.Cu) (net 9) (status 20))
 (segment (start 131.8 68.25) (end 131.8 66.2) (width 0.25) (layer F.Cu) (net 9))
 (segment (start 131.8 66.2) (end 137 61) (width 0.25) (layer F.Cu) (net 9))
 (segment (start 132.65 65.555) (end 132.65 65.35) (width 0.25) (layer B.Cu) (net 9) (status 30))
 (segment (start 132.65 65.35) (end 137 61) (width 0.25) (layer B.Cu) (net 9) (status 10))
 (segment (start 129.6543 67.7775) (end 131.3275 67.7775) (width 0.127) (layer F.Cu) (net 9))
 (segment (start 131.3275 67.7775) (end 131.8 68.25) (width 0.127) (layer F.Cu) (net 9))
 (segment (start 131.8 68.75) (end 132.85 68.75) (width 0.25) (layer F.Cu) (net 10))
 (segment (start 133.8 66.74) (end 137 63.54) (width 0.25) (layer F.Cu) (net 10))
 (segment (start 133.8 67.8) (end 133.8 66.74) (width 0.25) (layer F.Cu) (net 10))
 (segment (start 132.85 68.75) (end 133.8 67.8) (width 0.25) (layer F.Cu) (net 10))
 (segment (start 132.65 66.825) (end 133.715 66.825) (width 0.25) (layer B.Cu) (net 10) (status 10))
 (segment (start 133.715 66.825) (end 137 63.54) (width 0.25) (layer B.Cu) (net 10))
 (segment (start 132.65 66.825) (end 130.7 66.825) (width 0.6) (layer B.Cu) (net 10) (status 10))
 (segment (start 129.6543 68.4125) (end 130.6125 68.4125) (width 0.127) (layer F.Cu) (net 10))
 (segment (start 130.95 68.75) (end 131.8 68.75) (width 0.127) (layer F.Cu) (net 10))
 (segment (start 130.6125 68.4125) (end 130.95 68.75) (width 0.127) (layer F.Cu) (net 10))
 (segment (start 131.8 69.25) (end 133.83 69.25) (width 0.25) (layer F.Cu) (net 11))
 (segment (start 133.83 69.25) (end 137 66.08) (width 0.25) (layer F.Cu) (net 11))
 (segment (start 132.65 68.095) (end 134.985 68.095) (width 0.25) (layer B.Cu) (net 11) (status 10))
 (segment (start 134.985 68.095) (end 137 66.08) (width 0.25) (layer B.Cu) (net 11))
 (segment (start 132.65 68.095) (end 130.7 68.095) (width 0.6) (layer B.Cu) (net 11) (status 10))
 (segment (start 129.6543 69.0475) (end 130.8475 69.0475) (width 0.127) (layer F.Cu) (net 11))
 (segment (start 131.05 69.25) (end 131.8 69.25) (width 0.127) (layer F.Cu) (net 11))
 (segment (start 130.8475 69.0475) (end 131.05 69.25) (width 0.127) (layer F.Cu) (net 11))
 (segment (start 131.8 69.75) (end 135.87 69.75) (width 0.25) (layer F.Cu) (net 12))
 (segment (start 135.87 69.75) (end 137 68.62) (width 0.25) (layer F.Cu) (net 12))
 (segment (start 132.65 69.365) (end 136.255 69.365) (width 0.25) (layer B.Cu) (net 12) (status 10))
 (segment (start 136.255 69.365) (end 137 68.62) (width 0.25) (layer B.Cu) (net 12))
 (segment (start 132.65 69.365) (end 130.7 69.365) (width 0.6) (layer B.Cu) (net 12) (status 10))
 (segment (start 129.6543 69.6825) (end 131.7325 69.6825) (width 0.127) (layer F.Cu) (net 12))
 (segment (start 131.7325 69.6825) (end 131.8 69.75) (width 0.127) (layer F.Cu) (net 12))
 (segment (start 131.8 70.25) (end 136.09 70.25) (width 0.25) (layer F.Cu) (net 13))
 (segment (start 136.09 70.25) (end 137 71.16) (width 0.25) (layer F.Cu) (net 13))
 (segment (start 132.65 70.635) (end 136.475 70.635) (width 0.25) (layer B.Cu) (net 13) (status 10))
 (segment (start 136.475 70.635) (end 137 71.16) (width 0.25) (layer B.Cu) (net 13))
 (segment (start 132.65 70.635) (end 130.7 70.635) (width 0.6) (layer B.Cu) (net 13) (status 10))
 (segment (start 129.6543 70.3175) (end 131.7325 70.3175) (width 0.127) (layer F.Cu) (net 13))
 (segment (start 131.7325 70.3175) (end 131.8 70.25) (width 0.127) (layer F.Cu) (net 13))
 (segment (start 131.8 70.75) (end 134.05 70.75) (width 0.25) (layer F.Cu) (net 14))
 (segment (start 134.05 70.75) (end 137 73.7) (width 0.25) (layer F.Cu) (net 14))
 (segment (start 132.65 71.905) (end 135.205 71.905) (width 0.25) (layer B.Cu) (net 14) (status 10))
 (segment (start 135.205 71.905) (end 137 73.7) (width 0.25) (layer B.Cu) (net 14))
 (segment (start 132.65 71.905) (end 130.7 71.905) (width 0.6) (layer B.Cu) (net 14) (status 10))
 (segment (start 129.6543 70.9525) (end 130.8475 70.9525) (width 0.127) (layer F.Cu) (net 14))
 (segment (start 131.05 70.75) (end 131.8 70.75) (width 0.127) (layer F.Cu) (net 14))
 (segment (start 130.8475 70.9525) (end 131.05 70.75) (width 0.127) (layer F.Cu) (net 14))
 (segment (start 131.8 71.25) (end 132.85 71.25) (width 0.25) (layer F.Cu) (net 15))
 (segment (start 134 73.24) (end 137 76.24) (width 0.25) (layer F.Cu) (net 15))
 (segment (start 134 72.4) (end 134 73.24) (width 0.25) (layer F.Cu) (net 15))
 (segment (start 132.85 71.25) (end 134 72.4) (width 0.25) (layer F.Cu) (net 15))
 (segment (start 132.65 73.175) (end 133.935 73.175) (width 0.25) (layer B.Cu) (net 15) (status 10))
 (segment (start 133.935 73.175) (end 137 76.24) (width 0.25) (layer B.Cu) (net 15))
 (segment (start 132.65 73.175) (end 130.7 73.175) (width 0.6) (layer B.Cu) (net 15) (status 10))
 (segment (start 129.6543 71.5875) (end 130.6125 71.5875) (width 0.127) (layer F.Cu) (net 15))
 (segment (start 130.95 71.25) (end 131.8 71.25) (width 0.127) (layer F.Cu) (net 15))
 (segment (start 130.6125 71.5875) (end 130.95 71.25) (width 0.127) (layer F.Cu) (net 15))
 (segment (start 131.8 71.75) (end 131.8 73.58) (width 0.25) (layer F.Cu) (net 16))
 (segment (start 131.8 73.58) (end 137 78.78) (width 0.25) (layer F.Cu) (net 16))
 (segment (start 132.65 74.445) (end 132.665 74.445) (width 0.25) (layer B.Cu) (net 16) (status 30))
 (segment (start 132.665 74.445) (end 137 78.78) (width 0.25) (layer B.Cu) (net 16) (status 10))
 (segment (start 132.65 74.445) (end 130.7 74.445) (width 0.6) (layer B.Cu) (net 16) (status 10))
 (segment (start 129.6543 72.2225) (end 131.3275 72.2225) (width 0.127) (layer F.Cu) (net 16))
 (segment (start 131.3275 72.2225) (end 131.8 71.75) (width 0.127) (layer F.Cu) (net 16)))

